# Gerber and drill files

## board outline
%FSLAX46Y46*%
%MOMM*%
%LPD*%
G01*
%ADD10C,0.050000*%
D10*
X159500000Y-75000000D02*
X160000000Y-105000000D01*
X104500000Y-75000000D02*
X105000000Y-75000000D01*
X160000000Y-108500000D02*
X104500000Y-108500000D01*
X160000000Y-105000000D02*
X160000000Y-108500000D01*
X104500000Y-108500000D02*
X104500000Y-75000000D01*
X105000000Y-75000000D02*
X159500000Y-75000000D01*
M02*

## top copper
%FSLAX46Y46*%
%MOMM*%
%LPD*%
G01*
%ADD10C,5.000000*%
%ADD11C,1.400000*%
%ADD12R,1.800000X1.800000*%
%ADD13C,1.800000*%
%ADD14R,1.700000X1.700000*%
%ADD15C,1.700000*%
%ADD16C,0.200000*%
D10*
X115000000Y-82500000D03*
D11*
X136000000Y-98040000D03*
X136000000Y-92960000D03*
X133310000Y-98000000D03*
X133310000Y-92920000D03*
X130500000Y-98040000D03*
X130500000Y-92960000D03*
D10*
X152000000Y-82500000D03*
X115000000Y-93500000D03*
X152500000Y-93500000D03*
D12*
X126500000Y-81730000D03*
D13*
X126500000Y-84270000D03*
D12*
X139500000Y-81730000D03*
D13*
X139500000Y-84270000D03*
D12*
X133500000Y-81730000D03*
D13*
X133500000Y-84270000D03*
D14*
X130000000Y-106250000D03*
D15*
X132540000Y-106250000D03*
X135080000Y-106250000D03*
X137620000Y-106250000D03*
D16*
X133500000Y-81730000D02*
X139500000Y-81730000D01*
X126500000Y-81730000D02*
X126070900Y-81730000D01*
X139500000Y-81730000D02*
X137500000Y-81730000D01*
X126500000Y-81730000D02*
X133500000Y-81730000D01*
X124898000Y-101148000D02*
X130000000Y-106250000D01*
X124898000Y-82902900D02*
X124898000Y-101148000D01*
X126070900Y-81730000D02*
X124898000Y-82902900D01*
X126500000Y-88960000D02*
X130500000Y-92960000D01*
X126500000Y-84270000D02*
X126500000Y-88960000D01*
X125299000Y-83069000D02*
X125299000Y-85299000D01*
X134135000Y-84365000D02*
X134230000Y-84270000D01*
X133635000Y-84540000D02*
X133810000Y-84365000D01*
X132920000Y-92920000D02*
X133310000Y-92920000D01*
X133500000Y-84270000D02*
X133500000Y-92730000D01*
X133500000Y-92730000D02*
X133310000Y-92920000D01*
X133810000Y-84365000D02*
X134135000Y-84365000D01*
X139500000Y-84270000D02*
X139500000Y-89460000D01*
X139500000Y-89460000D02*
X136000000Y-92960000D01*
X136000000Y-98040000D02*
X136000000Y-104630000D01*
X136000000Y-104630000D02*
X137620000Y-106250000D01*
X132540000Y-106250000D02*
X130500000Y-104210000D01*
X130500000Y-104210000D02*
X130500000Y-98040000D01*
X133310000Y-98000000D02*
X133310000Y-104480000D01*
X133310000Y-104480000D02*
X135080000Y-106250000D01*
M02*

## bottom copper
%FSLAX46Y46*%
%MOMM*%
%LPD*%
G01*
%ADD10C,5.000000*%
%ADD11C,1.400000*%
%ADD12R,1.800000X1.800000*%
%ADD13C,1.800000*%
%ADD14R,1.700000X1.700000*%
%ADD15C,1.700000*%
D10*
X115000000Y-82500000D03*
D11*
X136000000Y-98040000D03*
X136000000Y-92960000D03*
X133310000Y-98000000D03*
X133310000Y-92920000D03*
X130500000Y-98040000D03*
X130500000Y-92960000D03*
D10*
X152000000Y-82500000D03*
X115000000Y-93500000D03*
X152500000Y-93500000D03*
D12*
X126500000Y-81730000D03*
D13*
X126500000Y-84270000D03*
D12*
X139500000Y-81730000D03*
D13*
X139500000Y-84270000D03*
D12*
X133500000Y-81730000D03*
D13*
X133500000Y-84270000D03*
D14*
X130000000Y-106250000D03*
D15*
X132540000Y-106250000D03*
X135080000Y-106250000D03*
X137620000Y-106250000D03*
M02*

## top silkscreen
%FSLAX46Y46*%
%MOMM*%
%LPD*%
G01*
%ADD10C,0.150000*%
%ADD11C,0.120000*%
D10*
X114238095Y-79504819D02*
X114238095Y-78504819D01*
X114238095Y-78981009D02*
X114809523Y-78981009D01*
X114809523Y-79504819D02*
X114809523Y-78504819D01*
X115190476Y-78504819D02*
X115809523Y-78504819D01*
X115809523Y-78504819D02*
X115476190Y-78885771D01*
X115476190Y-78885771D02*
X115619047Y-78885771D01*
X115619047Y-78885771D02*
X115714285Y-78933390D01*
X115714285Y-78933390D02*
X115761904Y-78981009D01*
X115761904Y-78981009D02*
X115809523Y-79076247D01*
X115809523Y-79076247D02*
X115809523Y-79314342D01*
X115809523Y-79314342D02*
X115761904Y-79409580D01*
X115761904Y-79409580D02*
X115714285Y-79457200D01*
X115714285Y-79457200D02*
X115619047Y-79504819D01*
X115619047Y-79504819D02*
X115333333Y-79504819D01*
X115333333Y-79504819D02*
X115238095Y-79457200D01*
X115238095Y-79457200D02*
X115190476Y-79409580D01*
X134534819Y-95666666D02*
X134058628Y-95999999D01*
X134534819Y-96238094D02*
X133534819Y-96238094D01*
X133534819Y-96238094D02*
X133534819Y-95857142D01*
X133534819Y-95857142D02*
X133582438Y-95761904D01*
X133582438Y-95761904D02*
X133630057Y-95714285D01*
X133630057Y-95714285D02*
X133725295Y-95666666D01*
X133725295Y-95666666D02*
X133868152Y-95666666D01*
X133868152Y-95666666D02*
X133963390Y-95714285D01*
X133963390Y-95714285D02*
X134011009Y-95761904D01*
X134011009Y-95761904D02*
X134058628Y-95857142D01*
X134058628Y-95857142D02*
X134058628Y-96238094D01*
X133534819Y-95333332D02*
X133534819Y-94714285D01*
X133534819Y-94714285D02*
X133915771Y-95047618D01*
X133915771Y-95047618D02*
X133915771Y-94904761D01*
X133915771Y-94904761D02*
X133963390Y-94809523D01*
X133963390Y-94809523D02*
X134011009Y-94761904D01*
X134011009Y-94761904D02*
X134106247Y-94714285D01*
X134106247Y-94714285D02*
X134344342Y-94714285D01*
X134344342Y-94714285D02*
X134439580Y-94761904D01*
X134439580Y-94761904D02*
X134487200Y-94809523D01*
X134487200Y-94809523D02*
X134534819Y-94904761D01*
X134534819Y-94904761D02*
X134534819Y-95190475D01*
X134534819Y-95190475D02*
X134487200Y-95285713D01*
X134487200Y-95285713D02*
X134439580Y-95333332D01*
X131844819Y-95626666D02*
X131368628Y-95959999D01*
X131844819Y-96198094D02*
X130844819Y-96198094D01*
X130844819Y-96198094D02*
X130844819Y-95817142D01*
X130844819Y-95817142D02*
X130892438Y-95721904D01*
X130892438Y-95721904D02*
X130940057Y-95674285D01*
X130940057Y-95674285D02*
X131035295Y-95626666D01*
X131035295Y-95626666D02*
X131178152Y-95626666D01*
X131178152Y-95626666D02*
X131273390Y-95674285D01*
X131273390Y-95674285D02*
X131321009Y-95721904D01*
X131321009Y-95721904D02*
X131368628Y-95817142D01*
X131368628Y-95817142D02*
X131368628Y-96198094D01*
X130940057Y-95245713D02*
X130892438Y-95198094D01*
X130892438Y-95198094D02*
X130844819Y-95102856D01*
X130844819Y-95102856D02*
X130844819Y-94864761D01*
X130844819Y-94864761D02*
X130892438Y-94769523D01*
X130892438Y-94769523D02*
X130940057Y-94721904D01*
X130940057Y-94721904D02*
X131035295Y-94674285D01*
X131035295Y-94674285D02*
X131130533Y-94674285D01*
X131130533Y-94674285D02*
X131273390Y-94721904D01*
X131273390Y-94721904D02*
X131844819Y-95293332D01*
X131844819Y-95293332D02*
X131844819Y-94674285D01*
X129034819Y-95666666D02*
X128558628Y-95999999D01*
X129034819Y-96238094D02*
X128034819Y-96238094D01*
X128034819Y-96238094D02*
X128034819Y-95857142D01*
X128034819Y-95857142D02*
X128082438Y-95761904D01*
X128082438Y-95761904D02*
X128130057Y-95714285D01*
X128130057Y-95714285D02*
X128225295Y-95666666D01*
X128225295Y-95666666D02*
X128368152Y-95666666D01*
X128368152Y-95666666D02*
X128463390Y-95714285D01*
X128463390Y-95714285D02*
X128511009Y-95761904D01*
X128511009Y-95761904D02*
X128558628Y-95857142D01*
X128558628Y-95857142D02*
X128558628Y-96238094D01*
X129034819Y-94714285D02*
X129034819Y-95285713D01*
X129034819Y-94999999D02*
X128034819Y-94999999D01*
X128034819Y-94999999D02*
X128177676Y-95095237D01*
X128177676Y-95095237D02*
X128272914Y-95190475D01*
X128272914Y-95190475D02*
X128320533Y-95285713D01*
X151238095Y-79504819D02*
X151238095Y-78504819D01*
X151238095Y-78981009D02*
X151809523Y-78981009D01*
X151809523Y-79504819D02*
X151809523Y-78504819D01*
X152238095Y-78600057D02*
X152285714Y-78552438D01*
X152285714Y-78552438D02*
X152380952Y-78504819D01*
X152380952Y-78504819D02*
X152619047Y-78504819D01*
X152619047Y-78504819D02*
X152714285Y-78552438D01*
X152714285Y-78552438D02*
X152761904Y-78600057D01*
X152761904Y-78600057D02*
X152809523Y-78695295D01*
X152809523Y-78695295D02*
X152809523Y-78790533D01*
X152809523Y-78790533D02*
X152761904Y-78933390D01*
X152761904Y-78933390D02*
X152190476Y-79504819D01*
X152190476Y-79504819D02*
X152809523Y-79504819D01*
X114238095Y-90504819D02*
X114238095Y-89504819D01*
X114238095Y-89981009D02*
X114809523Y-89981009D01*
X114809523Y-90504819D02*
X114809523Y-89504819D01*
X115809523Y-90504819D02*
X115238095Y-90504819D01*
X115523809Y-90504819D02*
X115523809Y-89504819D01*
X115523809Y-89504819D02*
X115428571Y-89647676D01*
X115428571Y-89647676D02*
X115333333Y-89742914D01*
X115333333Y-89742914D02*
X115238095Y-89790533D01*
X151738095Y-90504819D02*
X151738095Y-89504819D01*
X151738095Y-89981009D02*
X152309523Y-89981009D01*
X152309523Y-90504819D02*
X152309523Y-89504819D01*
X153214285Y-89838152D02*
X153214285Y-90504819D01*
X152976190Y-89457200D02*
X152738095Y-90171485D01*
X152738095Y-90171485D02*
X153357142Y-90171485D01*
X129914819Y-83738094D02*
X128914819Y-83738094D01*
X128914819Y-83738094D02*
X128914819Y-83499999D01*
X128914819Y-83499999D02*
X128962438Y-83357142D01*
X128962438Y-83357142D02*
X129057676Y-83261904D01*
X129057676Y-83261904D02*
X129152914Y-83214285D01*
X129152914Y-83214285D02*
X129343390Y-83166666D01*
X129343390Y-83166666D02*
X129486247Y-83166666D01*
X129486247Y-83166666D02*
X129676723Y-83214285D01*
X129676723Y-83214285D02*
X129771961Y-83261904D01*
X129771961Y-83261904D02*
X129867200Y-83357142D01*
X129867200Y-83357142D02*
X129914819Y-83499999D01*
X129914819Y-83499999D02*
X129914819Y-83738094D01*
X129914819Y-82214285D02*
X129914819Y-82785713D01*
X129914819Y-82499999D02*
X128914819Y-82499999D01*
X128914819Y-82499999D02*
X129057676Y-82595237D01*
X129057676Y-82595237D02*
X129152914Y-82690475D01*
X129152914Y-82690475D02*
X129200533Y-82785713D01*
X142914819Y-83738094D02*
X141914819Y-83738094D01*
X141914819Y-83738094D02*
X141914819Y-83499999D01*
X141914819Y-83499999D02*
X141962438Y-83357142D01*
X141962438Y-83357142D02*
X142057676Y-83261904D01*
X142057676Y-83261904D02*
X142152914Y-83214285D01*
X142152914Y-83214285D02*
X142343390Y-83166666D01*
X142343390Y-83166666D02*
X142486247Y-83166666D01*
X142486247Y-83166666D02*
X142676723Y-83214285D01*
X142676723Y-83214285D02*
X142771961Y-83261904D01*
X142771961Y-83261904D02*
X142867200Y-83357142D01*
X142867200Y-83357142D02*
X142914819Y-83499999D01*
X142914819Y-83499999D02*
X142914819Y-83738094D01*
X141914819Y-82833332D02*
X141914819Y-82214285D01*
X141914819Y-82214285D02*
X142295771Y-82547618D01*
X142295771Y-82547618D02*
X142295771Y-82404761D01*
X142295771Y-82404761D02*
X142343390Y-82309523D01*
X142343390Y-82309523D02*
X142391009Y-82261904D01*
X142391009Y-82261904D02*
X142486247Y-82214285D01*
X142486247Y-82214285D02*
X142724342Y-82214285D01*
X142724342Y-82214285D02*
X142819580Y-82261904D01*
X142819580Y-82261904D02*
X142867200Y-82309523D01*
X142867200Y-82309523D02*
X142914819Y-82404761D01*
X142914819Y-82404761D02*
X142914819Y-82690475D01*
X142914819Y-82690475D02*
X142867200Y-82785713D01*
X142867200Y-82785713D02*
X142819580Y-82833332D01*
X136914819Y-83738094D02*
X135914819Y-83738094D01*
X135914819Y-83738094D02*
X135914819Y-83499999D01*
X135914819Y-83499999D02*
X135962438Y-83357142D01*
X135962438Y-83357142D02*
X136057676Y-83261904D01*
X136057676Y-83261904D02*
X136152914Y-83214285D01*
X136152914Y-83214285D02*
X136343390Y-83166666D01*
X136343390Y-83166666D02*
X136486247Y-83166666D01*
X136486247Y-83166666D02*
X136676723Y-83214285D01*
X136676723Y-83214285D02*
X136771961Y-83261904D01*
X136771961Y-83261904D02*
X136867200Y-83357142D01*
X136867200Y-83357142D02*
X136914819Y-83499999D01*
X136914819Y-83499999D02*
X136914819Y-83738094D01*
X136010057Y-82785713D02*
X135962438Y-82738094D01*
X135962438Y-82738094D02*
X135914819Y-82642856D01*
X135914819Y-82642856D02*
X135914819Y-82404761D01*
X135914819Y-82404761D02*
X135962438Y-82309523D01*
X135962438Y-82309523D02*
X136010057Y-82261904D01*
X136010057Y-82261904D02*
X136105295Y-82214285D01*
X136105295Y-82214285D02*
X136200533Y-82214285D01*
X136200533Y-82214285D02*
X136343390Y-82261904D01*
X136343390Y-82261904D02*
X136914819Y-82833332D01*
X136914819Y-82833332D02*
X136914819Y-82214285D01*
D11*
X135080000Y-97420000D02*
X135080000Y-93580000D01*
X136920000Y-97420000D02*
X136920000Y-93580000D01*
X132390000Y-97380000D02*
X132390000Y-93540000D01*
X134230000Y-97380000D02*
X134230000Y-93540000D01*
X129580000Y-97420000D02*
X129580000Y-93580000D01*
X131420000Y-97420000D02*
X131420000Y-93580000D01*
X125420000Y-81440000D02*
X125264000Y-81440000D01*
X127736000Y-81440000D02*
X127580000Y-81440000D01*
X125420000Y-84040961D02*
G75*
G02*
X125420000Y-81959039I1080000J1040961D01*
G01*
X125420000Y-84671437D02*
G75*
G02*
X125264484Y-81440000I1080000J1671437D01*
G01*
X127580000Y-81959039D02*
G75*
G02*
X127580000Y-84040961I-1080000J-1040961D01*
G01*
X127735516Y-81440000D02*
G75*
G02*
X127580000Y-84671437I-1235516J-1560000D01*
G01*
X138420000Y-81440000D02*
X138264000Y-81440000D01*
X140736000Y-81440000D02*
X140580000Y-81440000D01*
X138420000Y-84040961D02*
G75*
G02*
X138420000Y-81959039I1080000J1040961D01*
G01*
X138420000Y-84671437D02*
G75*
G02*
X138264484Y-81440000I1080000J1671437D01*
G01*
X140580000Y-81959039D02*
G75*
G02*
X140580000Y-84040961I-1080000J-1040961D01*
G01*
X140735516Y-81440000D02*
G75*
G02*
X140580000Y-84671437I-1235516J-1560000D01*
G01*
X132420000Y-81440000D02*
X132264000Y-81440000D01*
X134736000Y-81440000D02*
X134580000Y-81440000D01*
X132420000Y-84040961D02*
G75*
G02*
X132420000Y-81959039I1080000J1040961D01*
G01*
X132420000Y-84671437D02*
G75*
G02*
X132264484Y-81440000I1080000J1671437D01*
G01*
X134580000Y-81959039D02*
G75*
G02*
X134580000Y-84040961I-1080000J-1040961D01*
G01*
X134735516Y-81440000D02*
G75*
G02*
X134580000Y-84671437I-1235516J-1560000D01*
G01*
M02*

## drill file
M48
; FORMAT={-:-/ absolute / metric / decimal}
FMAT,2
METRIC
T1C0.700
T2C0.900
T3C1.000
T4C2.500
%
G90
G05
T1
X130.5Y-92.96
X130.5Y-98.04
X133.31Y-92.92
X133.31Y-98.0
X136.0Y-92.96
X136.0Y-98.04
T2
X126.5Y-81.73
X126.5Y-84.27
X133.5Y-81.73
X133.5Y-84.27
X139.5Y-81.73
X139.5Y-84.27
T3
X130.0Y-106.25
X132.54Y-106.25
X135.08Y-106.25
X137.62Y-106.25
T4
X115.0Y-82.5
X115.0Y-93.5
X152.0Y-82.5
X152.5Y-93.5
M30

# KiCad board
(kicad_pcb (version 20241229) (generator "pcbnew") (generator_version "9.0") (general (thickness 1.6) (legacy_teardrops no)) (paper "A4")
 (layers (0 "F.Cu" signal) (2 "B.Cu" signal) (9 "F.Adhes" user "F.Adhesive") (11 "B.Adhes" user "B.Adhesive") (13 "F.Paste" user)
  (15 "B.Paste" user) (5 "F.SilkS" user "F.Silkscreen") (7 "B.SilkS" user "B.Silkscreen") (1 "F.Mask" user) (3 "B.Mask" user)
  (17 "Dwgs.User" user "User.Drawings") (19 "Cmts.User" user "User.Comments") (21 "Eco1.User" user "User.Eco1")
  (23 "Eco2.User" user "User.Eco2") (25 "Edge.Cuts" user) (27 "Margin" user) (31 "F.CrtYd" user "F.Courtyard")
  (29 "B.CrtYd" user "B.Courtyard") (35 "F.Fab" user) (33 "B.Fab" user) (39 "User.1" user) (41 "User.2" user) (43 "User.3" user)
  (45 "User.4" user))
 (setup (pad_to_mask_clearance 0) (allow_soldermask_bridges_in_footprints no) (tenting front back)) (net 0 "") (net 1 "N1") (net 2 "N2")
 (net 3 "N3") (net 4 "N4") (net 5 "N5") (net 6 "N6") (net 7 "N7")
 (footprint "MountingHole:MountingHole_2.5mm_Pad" (layer "F.Cu") (at 115 82.5)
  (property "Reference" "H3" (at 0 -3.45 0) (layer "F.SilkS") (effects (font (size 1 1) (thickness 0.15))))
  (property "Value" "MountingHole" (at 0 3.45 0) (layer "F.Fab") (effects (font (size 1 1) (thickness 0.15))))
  (pad "1" thru_hole circle (at 0 0) (size 5 5) (drill 2.5) (layers "*.Cu" "*.Mask") (remove_unused_layers no) (zone_connect 2)))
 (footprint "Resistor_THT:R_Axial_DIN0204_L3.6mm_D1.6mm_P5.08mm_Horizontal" (layer "F.Cu") (at 136 98.04 90)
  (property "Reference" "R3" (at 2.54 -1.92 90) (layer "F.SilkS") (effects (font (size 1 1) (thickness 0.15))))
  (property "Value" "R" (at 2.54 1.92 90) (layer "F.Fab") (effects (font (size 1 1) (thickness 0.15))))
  (fp_line (start 0.62 -0.92) (end 4.46 -0.92) (stroke (width 0.12) (type solid)) (layer "F.SilkS"))
  (fp_line (start 0.62 0.92) (end 4.46 0.92) (stroke (width 0.12) (type solid)) (layer "F.SilkS"))
  (pad "1" thru_hole circle (at 0 0 90) (size 1.4 1.4) (drill 0.7) (layers "*.Cu" "*.Mask") (remove_unused_layers no) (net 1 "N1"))
  (pad "2" thru_hole circle (at 5.08 0 90) (size 1.4 1.4) (drill 0.7) (layers "*.Cu" "*.Mask") (remove_unused_layers no) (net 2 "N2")))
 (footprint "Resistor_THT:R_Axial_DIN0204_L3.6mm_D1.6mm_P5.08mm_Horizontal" (layer "F.Cu") (at 133.31 98 90)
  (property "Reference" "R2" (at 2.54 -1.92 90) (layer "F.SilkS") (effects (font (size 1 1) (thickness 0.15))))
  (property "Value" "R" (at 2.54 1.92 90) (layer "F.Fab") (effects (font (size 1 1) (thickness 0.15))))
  (fp_line (start 0.62 -0.92) (end 4.46 -0.92) (stroke (width 0.12) (type solid)) (layer "F.SilkS"))
  (fp_line (start 0.62 0.92) (end 4.46 0.92) (stroke (width 0.12) (type solid)) (layer "F.SilkS"))
  (pad "1" thru_hole circle (at 0 0 90) (size 1.4 1.4) (drill 0.7) (layers "*.Cu" "*.Mask") (remove_unused_layers no) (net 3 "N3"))
  (pad "2" thru_hole circle (at 5.08 0 90) (size 1.4 1.4) (drill 0.7) (layers "*.Cu" "*.Mask") (remove_unused_layers no) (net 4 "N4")))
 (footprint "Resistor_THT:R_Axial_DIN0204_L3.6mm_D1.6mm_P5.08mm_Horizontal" (layer "F.Cu") (at 130.5 98.04 90)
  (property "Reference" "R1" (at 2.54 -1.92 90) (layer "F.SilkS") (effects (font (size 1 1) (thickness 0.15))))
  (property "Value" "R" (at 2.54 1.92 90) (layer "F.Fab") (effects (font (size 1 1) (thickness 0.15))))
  (fp_line (start 0.62 -0.92) (end 4.46 -0.92) (stroke (width 0.12) (type solid)) (layer "F.SilkS"))
  (fp_line (start 0.62 0.92) (end 4.46 0.92) (stroke (width 0.12) (type solid)) (layer "F.SilkS"))
  (pad "1" thru_hole circle (at 0 0 90) (size 1.4 1.4) (drill 0.7) (layers "*.Cu" "*.Mask") (remove_unused_layers no) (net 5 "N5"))
  (pad "2" thru_hole circle (at 5.08 0 90) (size 1.4 1.4) (drill 0.7) (layers "*.Cu" "*.Mask") (remove_unused_layers no) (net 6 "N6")))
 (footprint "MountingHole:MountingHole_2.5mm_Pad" (layer "F.Cu") (at 152 82.5)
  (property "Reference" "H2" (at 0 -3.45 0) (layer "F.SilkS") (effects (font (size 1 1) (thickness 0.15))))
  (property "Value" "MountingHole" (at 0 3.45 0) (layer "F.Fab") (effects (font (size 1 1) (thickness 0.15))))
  (pad "1" thru_hole circle (at 0 0) (size 5 5) (drill 2.5) (layers "*.Cu" "*.Mask") (remove_unused_layers no) (zone_connect 2)))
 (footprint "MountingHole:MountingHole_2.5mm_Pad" (layer "F.Cu") (at 115 93.5)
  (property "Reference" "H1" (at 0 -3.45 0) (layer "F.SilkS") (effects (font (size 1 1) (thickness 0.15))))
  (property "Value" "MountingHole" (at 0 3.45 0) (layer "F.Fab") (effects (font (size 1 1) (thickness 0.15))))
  (pad "1" thru_hole circle (at 0 0) (size 5 5) (drill 2.5) (layers "*.Cu" "*.Mask") (remove_unused_layers no) (zone_connect 2)))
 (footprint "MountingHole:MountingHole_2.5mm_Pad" (layer "F.Cu") (at 152.5 93.5)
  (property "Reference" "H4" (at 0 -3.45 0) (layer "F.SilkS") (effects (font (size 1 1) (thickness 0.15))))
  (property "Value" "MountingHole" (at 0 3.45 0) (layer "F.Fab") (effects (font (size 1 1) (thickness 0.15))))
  (pad "1" thru_hole circle (at 0 0) (size 5 5) (drill 2.5) (layers "*.Cu" "*.Mask") (remove_unused_layers no) (zone_connect 2)))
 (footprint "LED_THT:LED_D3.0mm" (layer "F.Cu") (at 126.5 81.73 -90)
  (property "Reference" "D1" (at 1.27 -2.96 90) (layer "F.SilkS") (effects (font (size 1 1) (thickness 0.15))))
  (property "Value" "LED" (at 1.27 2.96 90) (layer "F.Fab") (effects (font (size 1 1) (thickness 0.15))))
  (fp_line (start -0.29 1.08) (end -0.29 1.236) (stroke (width 0.12) (type solid)) (layer "F.SilkS"))
  (fp_line (start -0.29 -1.236) (end -0.29 -1.08) (stroke (width 0.12) (type solid)) (layer "F.SilkS"))
  (fp_arc (start 2.310961 1.08) (mid 1.27 1.5) (end 0.229039 1.08) (stroke (width 0.12) (type solid)) (layer "F.SilkS"))
  (fp_arc (start 2.941437 1.08) (mid 1.36566 1.987699) (end -0.29 1.235516) (stroke (width 0.12) (type solid)) (layer "F.SilkS"))
  (fp_arc (start 0.229039 -1.08) (mid 1.27 -1.5) (end 2.310961 -1.08) (stroke (width 0.12) (type solid)) (layer "F.SilkS"))
  (fp_arc (start -0.29 -1.235516) (mid 1.36566 -1.987699) (end 2.941437 -1.08) (stroke (width 0.12) (type solid)) (layer "F.SilkS"))
  (pad "1" thru_hole rect (at 0 0 270) (size 1.8 1.8) (drill 0.9) (layers "*.Cu" "*.Mask") (remove_unused_layers no) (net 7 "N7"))
  (pad "2" thru_hole circle (at 2.54 0 270) (size 1.8 1.8) (drill 0.9) (layers "*.Cu" "*.Mask") (remove_unused_layers no) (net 6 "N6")))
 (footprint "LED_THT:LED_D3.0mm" (layer "F.Cu") (at 139.5 81.73 -90)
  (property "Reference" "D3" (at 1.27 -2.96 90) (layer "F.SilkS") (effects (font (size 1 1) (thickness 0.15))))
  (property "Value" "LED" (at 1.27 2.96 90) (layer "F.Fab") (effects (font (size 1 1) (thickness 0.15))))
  (fp_line (start -0.29 1.08) (end -0.29 1.236) (stroke (width 0.12) (type solid)) (layer "F.SilkS"))
  (fp_line (start -0.29 -1.236) (end -0.29 -1.08) (stroke (width 0.12) (type solid)) (layer "F.SilkS"))
  (fp_arc (start 2.310961 1.08) (mid 1.27 1.5) (end 0.229039 1.08) (stroke (width 0.12) (type solid)) (layer "F.SilkS"))
  (fp_arc (start 2.941437 1.08) (mid 1.36566 1.987699) (end -0.29 1.235516) (stroke (width 0.12) (type solid)) (layer "F.SilkS"))
  (fp_arc (start 0.229039 -1.08) (mid 1.27 -1.5) (end 2.310961 -1.08) (stroke (width 0.12) (type solid)) (layer "F.SilkS"))
  (fp_arc (start -0.29 -1.235516) (mid 1.36566 -1.987699) (end 2.941437 -1.08) (stroke (width 0.12) (type solid)) (layer "F.SilkS"))
  (pad "1" thru_hole rect (at 0 0 270) (size 1.8 1.8) (drill 0.9) (layers "*.Cu" "*.Mask") (remove_unused_layers no) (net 7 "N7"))
  (pad "2" thru_hole circle (at 2.54 0 270) (size 1.8 1.8) (drill 0.9) (layers "*.Cu" "*.Mask") (remove_unused_layers no) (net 2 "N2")))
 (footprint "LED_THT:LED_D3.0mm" (layer "F.Cu") (at 133.5 81.73 -90)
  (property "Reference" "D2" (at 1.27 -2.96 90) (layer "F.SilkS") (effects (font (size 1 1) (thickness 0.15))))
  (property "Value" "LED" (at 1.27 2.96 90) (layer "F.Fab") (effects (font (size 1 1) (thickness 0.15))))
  (fp_line (start -0.29 1.08) (end -0.29 1.236) (stroke (width 0.12) (type solid)) (layer "F.SilkS"))
  (fp_line (start -0.29 -1.236) (end -0.29 -1.08) (stroke (width 0.12) (type solid)) (layer "F.SilkS"))
  (fp_arc (start 2.310961 1.08) (mid 1.27 1.5) (end 0.229039 1.08) (stroke (width 0.12) (type solid)) (layer "F.SilkS"))
  (fp_arc (start 2.941437 1.08) (mid 1.36566 1.987699) (end -0.29 1.235516) (stroke (width 0.12) (type solid)) (layer "F.SilkS"))
  (fp_arc (start 0.229039 -1.08) (mid 1.27 -1.5) (end 2.310961 -1.08) (stroke (width 0.12) (type solid)) (layer "F.SilkS"))
  (fp_arc (start -0.29 -1.235516) (mid 1.36566 -1.987699) (end 2.941437 -1.08) (stroke (width 0.12) (type solid)) (layer "F.SilkS"))
  (pad "1" thru_hole rect (at 0 0 270) (size 1.8 1.8) (drill 0.9) (layers "*.Cu" "*.Mask") (remove_unused_layers no) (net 7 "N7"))
  (pad "2" thru_hole circle (at 2.54 0 270) (size 1.8 1.8) (drill 0.9) (layers "*.Cu" "*.Mask") (remove_unused_layers no) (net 4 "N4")))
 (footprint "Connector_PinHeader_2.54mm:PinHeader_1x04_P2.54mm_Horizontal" (layer "B.Cu") (at 130 106.25 -90)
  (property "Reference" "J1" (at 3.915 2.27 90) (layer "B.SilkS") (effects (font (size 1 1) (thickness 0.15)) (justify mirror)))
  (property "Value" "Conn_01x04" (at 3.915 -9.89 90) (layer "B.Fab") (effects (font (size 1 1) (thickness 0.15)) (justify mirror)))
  (pad "1" thru_hole rect (at 0 0 270) (size 1.7 1.7) (drill 1) (layers "*.Cu" "*.Mask") (remove_unused_layers no) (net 7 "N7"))
  (pad "2" thru_hole circle (at 0 -2.54 270) (size 1.7 1.7) (drill 1) (layers "*.Cu" "*.Mask") (remove_unused_layers no) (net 5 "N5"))
  (pad "3" thru_hole circle (at 0 -5.08 270) (size 1.7 1.7) (drill 1) (layers "*.Cu" "*.Mask") (remove_unused_layers no) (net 3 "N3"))
  (pad "4" thru_hole circle (at 0 -7.62 270) (size 1.7 1.7) (drill 1) (layers "*.Cu" "*.Mask") (remove_unused_layers no) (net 1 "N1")))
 (gr_line (start 159.5 75) (end 160 105) (stroke (width 0.05) (type default)) (layer "Edge.Cuts"))
 (gr_line (start 104.5 75) (end 105 75) (stroke (width 0.05) (type default)) (layer "Edge.Cuts"))
 (gr_line (start 160 108.5) (end 104.5 108.5) (stroke (width 0.05) (type default)) (layer "Edge.Cuts"))
 (gr_line (start 160 105) (end 160 108.5) (stroke (width 0.05) (type default)) (layer "Edge.Cuts"))
 (gr_line (start 104.5 108.5) (end 104.5 75) (stroke (width 0.05) (type default)) (layer "Edge.Cuts"))
 (gr_line (start 105 75) (end 159.5 75) (stroke (width 0.05) (type default)) (layer "Edge.Cuts"))
 (segment (start 133.5 81.73) (end 139.5 81.73) (width 0.2) (layer "F.Cu") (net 7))
 (segment (start 126.5 81.73) (end 126.0709 81.73) (width 0.2) (layer "F.Cu") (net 7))
 (segment (start 139.5 81.73) (end 137.5 81.73) (width 0.2) (layer "F.Cu") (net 7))
 (segment (start 126.5 81.73) (end 133.5 81.73) (width 0.2) (layer "F.Cu") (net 7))
 (segment (start 124.898 101.148) (end 130 106.25) (width 0.2) (layer "F.Cu") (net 7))
 (segment (start 124.898 82.9029) (end 124.898 101.148) (width 0.2) (layer "F.Cu") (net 7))
 (segment (start 126.0709 81.73) (end 124.898 82.9029) (width 0.2) (layer "F.Cu") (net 7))
 (segment (start 126.5 88.96) (end 130.5 92.96) (width 0.2) (layer "F.Cu") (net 6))
 (segment (start 126.5 84.27) (end 126.5 88.96) (width 0.2) (layer "F.Cu") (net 6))
 (segment (start 125.299 83.069) (end 125.299 85.299) (width 0.2) (layer "F.Cu") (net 4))
 (segment (start 134.135 84.365) (end 134.23 84.27) (width 0.2) (layer "F.Cu") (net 4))
 (segment (start 133.635 84.54) (end 133.81 84.365) (width 0.2) (layer "F.Cu") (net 4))
 (segment (start 132.92 92.92) (end 133.31 92.92) (width 0.2) (layer "F.Cu") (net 4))
 (segment (start 133.5 84.27) (end 133.5 92.73) (width 0.2) (layer "F.Cu") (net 4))
 (segment (start 133.5 92.73) (end 133.31 92.92) (width 0.2) (layer "F.Cu") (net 4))
 (segment (start 133.81 84.365) (end 134.135 84.365) (width 0.2) (layer "F.Cu") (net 4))
 (segment (start 139.5 84.27) (end 139.5 89.46) (width 0.2) (layer "F.Cu") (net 2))
 (segment (start 139.5 89.46) (end 136 92.96) (width 0.2) (layer "F.Cu") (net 2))
 (segment (start 136 98.04) (end 136 104.63) (width 0.2) (layer "F.Cu") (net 1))
 (segment (start 136 104.63) (end 137.62 106.25) (width 0.2) (layer "F.Cu") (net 1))
 (segment (start 132.54 106.25) (end 130.5 104.21) (width 0.2) (layer "F.Cu") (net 5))
 (segment (start 130.5 104.21) (end 130.5 98.04) (width 0.2) (layer "F.Cu") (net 5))
 (segment (start 133.31 98) (end 133.31 104.48) (width 0.2) (layer "F.Cu") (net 3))
 (segment (start 133.31 104.48) (end 135.08 106.25) (width 0.2) (layer "F.Cu") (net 3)))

